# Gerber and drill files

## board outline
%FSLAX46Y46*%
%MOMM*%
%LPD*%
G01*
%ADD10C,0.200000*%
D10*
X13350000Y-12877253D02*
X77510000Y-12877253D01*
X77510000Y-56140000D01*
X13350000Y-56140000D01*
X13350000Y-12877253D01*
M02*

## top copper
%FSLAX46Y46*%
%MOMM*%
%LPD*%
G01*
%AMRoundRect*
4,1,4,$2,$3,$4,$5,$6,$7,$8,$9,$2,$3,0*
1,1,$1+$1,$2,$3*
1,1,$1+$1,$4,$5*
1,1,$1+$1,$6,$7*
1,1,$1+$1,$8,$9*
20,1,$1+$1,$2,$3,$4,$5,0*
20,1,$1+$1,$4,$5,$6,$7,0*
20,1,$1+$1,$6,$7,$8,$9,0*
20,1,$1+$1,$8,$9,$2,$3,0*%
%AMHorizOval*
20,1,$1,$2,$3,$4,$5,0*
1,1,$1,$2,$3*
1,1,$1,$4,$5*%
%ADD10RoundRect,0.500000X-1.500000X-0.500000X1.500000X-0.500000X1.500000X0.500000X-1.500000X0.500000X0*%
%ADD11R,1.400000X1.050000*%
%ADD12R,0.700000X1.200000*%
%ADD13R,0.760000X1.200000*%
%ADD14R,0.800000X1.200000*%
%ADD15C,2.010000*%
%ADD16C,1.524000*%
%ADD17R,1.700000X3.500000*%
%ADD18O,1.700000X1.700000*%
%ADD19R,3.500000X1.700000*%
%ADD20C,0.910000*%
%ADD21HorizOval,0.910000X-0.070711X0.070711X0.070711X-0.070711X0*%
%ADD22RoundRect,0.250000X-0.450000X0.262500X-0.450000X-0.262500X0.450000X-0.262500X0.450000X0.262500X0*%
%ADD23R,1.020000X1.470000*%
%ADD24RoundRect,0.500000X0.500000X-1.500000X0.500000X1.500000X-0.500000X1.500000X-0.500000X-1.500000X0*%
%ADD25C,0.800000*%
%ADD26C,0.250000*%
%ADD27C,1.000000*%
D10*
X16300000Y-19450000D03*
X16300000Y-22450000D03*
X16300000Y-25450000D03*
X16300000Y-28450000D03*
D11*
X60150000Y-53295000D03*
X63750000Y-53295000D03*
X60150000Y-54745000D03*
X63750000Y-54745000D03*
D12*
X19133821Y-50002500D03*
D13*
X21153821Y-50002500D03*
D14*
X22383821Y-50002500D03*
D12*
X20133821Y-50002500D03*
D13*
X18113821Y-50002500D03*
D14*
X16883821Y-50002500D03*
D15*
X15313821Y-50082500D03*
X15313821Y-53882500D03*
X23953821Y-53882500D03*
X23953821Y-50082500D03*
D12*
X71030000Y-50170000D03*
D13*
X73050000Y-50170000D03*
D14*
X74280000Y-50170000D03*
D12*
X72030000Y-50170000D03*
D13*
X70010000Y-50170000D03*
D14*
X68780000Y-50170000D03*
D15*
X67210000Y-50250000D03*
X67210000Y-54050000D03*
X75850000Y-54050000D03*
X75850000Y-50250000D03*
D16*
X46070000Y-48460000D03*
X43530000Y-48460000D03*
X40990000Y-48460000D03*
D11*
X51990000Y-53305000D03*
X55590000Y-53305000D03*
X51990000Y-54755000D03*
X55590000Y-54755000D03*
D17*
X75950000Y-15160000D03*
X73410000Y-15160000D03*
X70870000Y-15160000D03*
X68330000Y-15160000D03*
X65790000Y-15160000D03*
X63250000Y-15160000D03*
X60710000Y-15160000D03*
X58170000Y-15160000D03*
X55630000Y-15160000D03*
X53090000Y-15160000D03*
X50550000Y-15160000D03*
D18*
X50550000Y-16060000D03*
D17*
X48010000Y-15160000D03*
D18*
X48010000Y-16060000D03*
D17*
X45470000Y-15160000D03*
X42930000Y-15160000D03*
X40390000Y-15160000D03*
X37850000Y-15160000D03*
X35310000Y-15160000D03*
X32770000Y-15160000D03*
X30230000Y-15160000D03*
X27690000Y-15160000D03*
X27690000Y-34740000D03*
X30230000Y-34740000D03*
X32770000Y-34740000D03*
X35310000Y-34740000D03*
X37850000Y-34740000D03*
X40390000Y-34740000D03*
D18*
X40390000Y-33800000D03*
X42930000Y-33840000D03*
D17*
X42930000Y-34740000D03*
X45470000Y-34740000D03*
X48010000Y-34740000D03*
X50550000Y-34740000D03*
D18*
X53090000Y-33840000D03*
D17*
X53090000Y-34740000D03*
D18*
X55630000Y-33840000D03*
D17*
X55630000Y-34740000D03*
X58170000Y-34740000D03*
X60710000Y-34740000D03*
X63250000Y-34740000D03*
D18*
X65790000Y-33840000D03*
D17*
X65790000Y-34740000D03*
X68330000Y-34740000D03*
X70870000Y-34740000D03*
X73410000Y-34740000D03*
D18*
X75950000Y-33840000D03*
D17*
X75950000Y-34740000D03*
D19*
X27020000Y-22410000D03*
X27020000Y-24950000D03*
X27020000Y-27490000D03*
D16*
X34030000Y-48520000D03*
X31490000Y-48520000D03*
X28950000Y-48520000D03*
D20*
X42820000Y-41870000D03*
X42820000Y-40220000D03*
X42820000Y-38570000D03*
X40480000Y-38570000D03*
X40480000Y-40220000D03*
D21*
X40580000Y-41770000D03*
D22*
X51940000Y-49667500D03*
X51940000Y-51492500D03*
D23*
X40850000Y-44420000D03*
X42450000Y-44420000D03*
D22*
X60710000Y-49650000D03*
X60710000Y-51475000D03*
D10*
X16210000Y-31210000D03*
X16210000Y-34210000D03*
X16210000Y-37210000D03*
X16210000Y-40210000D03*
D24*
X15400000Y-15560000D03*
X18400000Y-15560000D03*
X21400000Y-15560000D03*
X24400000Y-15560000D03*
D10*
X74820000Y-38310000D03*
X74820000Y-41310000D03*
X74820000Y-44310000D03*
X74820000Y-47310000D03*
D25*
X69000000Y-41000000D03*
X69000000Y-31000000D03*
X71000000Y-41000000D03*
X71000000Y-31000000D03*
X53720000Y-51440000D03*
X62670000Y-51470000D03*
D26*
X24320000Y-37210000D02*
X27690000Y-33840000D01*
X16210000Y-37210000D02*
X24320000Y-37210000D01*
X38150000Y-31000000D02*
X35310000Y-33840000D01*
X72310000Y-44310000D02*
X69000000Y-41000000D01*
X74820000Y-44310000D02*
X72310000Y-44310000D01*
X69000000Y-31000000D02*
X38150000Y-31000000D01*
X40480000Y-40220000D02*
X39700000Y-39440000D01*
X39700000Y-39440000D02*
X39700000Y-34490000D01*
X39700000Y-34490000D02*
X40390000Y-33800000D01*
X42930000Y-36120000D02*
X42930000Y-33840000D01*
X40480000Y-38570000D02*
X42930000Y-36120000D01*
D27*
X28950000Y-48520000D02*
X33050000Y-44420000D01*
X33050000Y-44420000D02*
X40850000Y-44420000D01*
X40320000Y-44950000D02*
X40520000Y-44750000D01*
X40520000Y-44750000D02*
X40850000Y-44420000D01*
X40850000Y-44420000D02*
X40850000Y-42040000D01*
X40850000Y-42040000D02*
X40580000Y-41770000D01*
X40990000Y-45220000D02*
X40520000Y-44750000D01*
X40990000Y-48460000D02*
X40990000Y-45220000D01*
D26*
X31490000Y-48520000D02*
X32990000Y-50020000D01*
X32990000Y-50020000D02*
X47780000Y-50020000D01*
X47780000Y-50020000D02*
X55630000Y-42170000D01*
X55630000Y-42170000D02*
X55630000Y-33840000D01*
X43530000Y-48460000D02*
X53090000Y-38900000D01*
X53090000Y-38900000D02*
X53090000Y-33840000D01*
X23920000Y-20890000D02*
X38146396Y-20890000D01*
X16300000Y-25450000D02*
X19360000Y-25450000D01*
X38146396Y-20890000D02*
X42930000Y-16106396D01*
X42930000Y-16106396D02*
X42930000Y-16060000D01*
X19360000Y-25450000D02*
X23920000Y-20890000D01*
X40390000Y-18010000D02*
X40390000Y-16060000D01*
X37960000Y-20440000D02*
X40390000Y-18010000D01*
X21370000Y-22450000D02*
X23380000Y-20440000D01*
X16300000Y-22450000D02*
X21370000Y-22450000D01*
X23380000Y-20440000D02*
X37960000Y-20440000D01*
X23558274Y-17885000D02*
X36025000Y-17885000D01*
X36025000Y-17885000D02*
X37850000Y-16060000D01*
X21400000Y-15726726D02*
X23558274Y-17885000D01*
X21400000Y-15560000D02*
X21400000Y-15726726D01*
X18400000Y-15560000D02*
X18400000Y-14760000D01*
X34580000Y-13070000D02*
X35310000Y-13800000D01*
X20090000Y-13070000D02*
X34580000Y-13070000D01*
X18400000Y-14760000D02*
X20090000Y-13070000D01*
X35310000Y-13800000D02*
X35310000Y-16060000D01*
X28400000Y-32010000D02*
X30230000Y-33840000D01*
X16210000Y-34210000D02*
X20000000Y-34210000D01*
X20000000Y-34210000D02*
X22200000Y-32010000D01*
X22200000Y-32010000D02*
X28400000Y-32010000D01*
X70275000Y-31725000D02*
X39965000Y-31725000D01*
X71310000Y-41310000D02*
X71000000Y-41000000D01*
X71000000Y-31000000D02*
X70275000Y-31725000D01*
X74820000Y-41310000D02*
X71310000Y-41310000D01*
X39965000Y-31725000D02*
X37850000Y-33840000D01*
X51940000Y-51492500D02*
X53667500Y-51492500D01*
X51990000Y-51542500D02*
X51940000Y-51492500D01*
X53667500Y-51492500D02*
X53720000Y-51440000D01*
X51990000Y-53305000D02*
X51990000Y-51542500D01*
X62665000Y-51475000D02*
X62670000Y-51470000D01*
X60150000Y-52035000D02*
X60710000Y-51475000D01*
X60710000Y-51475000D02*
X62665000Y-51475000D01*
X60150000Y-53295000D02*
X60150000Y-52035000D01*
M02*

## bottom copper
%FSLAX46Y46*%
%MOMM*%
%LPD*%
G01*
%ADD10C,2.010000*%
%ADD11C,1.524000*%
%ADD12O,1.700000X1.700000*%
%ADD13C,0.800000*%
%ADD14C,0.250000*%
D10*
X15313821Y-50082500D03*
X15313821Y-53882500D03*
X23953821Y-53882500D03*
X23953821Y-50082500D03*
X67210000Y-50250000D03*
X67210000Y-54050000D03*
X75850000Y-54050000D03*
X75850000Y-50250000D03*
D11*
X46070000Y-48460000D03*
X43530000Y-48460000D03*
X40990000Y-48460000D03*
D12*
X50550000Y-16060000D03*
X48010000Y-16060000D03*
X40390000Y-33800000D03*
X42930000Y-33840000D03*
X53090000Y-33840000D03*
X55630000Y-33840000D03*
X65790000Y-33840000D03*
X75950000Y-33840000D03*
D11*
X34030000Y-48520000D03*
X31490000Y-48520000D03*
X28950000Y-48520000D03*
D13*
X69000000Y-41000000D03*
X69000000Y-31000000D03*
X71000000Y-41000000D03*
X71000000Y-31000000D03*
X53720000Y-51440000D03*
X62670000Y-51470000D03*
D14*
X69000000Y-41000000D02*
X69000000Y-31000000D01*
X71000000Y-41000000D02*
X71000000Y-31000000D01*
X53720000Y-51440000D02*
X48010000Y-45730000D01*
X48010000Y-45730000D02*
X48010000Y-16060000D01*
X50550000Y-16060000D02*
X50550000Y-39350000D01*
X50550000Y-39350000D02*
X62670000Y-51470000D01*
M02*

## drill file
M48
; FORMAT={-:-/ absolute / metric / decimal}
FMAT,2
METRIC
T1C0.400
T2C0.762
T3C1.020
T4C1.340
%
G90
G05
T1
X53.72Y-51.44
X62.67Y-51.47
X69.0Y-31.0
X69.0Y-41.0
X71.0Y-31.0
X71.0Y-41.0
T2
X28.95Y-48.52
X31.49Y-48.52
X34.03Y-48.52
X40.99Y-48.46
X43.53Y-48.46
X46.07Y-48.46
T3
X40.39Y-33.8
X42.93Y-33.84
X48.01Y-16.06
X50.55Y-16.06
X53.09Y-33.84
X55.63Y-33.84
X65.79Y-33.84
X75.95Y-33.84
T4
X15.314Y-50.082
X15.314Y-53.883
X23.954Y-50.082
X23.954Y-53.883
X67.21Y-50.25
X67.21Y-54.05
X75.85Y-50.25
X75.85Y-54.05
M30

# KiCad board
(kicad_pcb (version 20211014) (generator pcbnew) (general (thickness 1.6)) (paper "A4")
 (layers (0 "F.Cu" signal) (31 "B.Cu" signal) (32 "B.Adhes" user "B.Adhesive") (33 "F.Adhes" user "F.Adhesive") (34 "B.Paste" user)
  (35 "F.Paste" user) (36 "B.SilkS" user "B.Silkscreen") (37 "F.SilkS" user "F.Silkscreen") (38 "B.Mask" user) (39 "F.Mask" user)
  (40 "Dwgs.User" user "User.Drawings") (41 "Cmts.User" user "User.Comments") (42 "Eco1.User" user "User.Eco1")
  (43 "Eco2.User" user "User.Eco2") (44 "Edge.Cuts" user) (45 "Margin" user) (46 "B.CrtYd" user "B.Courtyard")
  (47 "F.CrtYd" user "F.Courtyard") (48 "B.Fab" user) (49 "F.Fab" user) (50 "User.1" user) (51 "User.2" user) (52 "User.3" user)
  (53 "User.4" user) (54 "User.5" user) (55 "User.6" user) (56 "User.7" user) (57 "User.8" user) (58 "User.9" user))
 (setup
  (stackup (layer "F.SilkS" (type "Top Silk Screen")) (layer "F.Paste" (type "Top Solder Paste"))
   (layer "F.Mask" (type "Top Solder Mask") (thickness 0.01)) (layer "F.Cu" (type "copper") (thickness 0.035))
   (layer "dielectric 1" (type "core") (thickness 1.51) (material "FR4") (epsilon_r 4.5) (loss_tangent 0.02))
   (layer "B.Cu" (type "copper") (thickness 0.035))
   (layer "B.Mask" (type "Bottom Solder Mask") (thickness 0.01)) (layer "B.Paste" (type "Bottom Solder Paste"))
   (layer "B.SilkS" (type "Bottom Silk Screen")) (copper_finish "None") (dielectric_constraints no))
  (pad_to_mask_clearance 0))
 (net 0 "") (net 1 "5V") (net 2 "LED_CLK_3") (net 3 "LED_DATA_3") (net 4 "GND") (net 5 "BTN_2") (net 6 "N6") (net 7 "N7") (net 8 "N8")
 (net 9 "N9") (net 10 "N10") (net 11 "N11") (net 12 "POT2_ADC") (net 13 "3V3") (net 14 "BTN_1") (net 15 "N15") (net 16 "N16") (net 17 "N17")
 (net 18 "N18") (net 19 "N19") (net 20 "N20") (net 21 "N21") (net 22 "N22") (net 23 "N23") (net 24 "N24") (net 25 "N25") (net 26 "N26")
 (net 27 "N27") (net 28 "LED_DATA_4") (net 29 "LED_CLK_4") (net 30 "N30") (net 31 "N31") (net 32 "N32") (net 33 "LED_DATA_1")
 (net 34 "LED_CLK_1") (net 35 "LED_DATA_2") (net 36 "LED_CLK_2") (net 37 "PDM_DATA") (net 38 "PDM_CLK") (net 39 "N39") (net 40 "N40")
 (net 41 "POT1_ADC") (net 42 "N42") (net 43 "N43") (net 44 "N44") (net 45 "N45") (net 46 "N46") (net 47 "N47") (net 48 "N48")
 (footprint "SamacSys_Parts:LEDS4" (layer "F.Cu") (at 16.3 19.45)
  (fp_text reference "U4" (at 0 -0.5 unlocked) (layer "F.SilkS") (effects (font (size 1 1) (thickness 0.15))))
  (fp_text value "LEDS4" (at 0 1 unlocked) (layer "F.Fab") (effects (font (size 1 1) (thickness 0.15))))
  (pad "1" smd roundrect (at 0 0) (size 4 2) (layers "F.Cu" "F.Paste" "F.Mask") (roundrect_rratio 0.25) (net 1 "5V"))
  (pad "2" smd roundrect (at 0 3) (size 4 2) (layers "F.Cu" "F.Paste" "F.Mask") (roundrect_rratio 0.25) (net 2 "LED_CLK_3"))
  (pad "3" smd roundrect (at 0 6) (size 4 2) (layers "F.Cu" "F.Paste" "F.Mask") (roundrect_rratio 0.25) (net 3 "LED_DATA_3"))
  (pad "4" smd roundrect (at 0 9) (size 4 2) (layers "F.Cu" "F.Paste" "F.Mask") (roundrect_rratio 0.25) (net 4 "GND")))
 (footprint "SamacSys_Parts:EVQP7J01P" (layer "F.Cu") (at 61.65 54.02)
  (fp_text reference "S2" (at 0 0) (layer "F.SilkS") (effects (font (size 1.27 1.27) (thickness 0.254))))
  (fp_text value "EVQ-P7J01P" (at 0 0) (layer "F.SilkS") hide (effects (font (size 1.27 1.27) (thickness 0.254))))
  (pad "1" smd rect locked (at -1.5 -0.725 90) (size 1.05 1.4) (layers "F.Cu" "F.Paste" "F.Mask") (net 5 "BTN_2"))
  (pad "2" smd rect locked (at 2.1 -0.725 90) (size 1.05 1.4) (layers "F.Cu" "F.Paste" "F.Mask") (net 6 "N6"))
  (pad "3" smd rect locked (at -1.5 0.725 90) (size 1.05 1.4) (layers "F.Cu" "F.Paste" "F.Mask") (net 4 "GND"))
  (pad "4" smd rect locked (at 2.1 0.725 90) (size 1.05 1.4) (layers "F.Cu" "F.Paste" "F.Mask") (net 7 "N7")))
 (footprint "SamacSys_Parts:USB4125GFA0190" (layer "F.Cu") (at 19.633821 53.0825)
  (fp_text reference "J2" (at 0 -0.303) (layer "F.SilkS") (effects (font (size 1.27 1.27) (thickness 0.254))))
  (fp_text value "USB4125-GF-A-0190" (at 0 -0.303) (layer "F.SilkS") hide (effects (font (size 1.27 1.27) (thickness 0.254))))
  (pad "A5" smd rect locked (at -0.5 -3.08) (size 0.7 1.2) (layers "F.Cu" "F.Paste" "F.Mask") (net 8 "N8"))
  (pad "A9" smd rect locked (at 1.52 -3.08) (size 0.76 1.2) (layers "F.Cu" "F.Paste" "F.Mask") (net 1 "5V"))
  (pad "A12" smd rect locked (at 2.75 -3.08) (size 0.8 1.2) (layers "F.Cu" "F.Paste" "F.Mask") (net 4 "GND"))
  (pad "B5" smd rect locked (at 0.5 -3.08) (size 0.7 1.2) (layers "F.Cu" "F.Paste" "F.Mask") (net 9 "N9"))
  (pad "B9" smd rect locked (at -1.52 -3.08) (size 0.76 1.2) (layers "F.Cu" "F.Paste" "F.Mask") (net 1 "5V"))
  (pad "B12" smd rect locked (at -2.75 -3.08) (size 0.8 1.2) (layers "F.Cu" "F.Paste" "F.Mask") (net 4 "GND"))
  (pad "MH1" thru_hole circle locked (at -4.32 -3) (size 2.01 2.01) (drill 1.34) (layers *.Cu *.Mask) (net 4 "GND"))
  (pad "MH2" thru_hole circle locked (at -4.32 0.8) (size 2.01 2.01) (drill 1.34) (layers *.Cu *.Mask) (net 4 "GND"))
  (pad "MH3" thru_hole circle locked (at 4.32 0.8) (size 2.01 2.01) (drill 1.34) (layers *.Cu *.Mask) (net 4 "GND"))
  (pad "MH4" thru_hole circle locked (at 4.32 -3) (size 2.01 2.01) (drill 1.34) (layers *.Cu *.Mask) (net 4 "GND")))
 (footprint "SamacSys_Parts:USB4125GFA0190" (layer "F.Cu") (at 71.53 53.25)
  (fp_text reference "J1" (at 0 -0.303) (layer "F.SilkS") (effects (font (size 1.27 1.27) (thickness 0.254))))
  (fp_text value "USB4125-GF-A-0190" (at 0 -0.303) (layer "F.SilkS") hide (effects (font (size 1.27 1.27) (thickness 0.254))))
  (pad "A5" smd rect locked (at -0.5 -3.08) (size 0.7 1.2) (layers "F.Cu" "F.Paste" "F.Mask") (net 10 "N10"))
  (pad "A9" smd rect locked (at 1.52 -3.08) (size 0.76 1.2) (layers "F.Cu" "F.Paste" "F.Mask") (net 1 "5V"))
  (pad "A12" smd rect locked (at 2.75 -3.08) (size 0.8 1.2) (layers "F.Cu" "F.Paste" "F.Mask") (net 4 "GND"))
  (pad "B5" smd rect locked (at 0.5 -3.08) (size 0.7 1.2) (layers "F.Cu" "F.Paste" "F.Mask") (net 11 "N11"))
  (pad "B9" smd rect locked (at -1.52 -3.08) (size 0.76 1.2) (layers "F.Cu" "F.Paste" "F.Mask") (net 1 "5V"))
  (pad "B12" smd rect locked (at -2.75 -3.08) (size 0.8 1.2) (layers "F.Cu" "F.Paste" "F.Mask") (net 4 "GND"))
  (pad "MH1" thru_hole circle locked (at -4.32 -3) (size 2.01 2.01) (drill 1.34) (layers *.Cu *.Mask) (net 4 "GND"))
  (pad "MH2" thru_hole circle locked (at -4.32 0.8) (size 2.01 2.01) (drill 1.34) (layers *.Cu *.Mask) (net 4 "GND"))
  (pad "MH3" thru_hole circle locked (at 4.32 0.8) (size 2.01 2.01) (drill 1.34) (layers *.Cu *.Mask) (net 4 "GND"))
  (pad "MH4" thru_hole circle locked (at 4.32 -3) (size 2.01 2.01) (drill 1.34) (layers *.Cu *.Mask) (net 4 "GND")))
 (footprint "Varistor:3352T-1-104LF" (layer "F.Cu") (at 43.53 48.46 180)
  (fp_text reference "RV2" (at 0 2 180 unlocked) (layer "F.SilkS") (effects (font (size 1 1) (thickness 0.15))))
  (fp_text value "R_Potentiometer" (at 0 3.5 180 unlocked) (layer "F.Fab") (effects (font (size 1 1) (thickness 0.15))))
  (pad "1" thru_hole circle (at -2.54 0 180) (size 1.524 1.524) (drill 0.762) (layers *.Cu *.Mask) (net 4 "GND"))
  (pad "2" thru_hole circle (at 0 0 180) (size 1.524 1.524) (drill 0.762) (layers *.Cu *.Mask) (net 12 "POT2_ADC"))
  (pad "3" thru_hole circle (at 2.54 0 180) (size 1.524 1.524) (drill 0.762) (layers *.Cu *.Mask) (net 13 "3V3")))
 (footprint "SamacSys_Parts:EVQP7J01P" (layer "F.Cu") (at 53.49 54.03)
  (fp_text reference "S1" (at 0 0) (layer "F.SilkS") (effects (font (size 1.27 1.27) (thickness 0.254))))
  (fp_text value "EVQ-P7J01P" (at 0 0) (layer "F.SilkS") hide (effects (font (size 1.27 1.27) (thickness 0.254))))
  (pad "1" smd rect locked (at -1.5 -0.725 90) (size 1.05 1.4) (layers "F.Cu" "F.Paste" "F.Mask") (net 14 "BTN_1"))
  (pad "2" smd rect locked (at 2.1 -0.725 90) (size 1.05 1.4) (layers "F.Cu" "F.Paste" "F.Mask") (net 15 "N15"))
  (pad "3" smd rect locked (at -1.5 0.725 90) (size 1.05 1.4) (layers "F.Cu" "F.Paste" "F.Mask") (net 4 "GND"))
  (pad "4" smd rect locked (at 2.1 0.725 90) (size 1.05 1.4) (layers "F.Cu" "F.Paste" "F.Mask") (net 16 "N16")))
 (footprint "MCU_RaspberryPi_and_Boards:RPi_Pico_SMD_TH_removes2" (layer "F.Cu") (at 51.82 24.95 -90)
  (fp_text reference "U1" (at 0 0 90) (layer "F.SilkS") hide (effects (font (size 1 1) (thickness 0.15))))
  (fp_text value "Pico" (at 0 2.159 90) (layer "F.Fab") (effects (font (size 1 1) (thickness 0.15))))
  (pad "1" smd rect (at -8.89 -24.13 270) (size 3.5 1.7) (drill (offset -0.9 0)) (layers "F.Cu" "F.Mask") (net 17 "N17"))
  (pad "2" smd rect (at -8.89 -21.59 270) (size 3.5 1.7) (drill (offset -0.9 0)) (layers "F.Cu" "F.Mask") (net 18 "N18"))
  (pad "3" smd rect (at -8.89 -19.05 270) (size 3.5 1.7) (drill (offset -0.9 0)) (layers "F.Cu" "F.Mask") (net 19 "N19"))
  (pad "4" smd rect (at -8.89 -16.51 270) (size 3.5 1.7) (drill (offset -0.9 0)) (layers "F.Cu" "F.Mask") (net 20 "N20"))
  (pad "5" smd rect (at -8.89 -13.97 270) (size 3.5 1.7) (drill (offset -0.9 0)) (layers "F.Cu" "F.Mask") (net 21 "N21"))
  (pad "6" smd rect (at -8.89 -11.43 270) (size 3.5 1.7) (drill (offset -0.9 0)) (layers "F.Cu" "F.Mask") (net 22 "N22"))
  (pad "7" smd rect (at -8.89 -8.89 270) (size 3.5 1.7) (drill (offset -0.9 0)) (layers "F.Cu" "F.Mask") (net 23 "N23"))
  (pad "8" smd rect (at -8.89 -6.35 270) (size 3.5 1.7) (drill (offset -0.9 0)) (layers "F.Cu" "F.Mask") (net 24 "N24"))
  (pad "9" smd rect (at -8.89 -3.81 270) (size 3.5 1.7) (drill (offset -0.9 0)) (layers "F.Cu" "F.Mask") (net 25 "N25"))
  (pad "10" smd rect (at -8.89 -1.27 270) (size 3.5 1.7) (drill (offset -0.9 0)) (layers "F.Cu" "F.Mask") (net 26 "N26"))
  (pad "11" smd rect (at -8.89 1.27 270) (size 3.5 1.7) (drill (offset -0.9 0)) (layers "F.Cu" "F.Mask") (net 5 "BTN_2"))
  (pad "11" thru_hole oval (at -8.89 1.27 270) (size 1.7 1.7) (drill 1.02) (layers *.Cu *.Mask) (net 5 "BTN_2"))
  (pad "12" smd rect (at -8.89 3.81 270) (size 3.5 1.7) (drill (offset -0.9 0)) (layers "F.Cu" "F.Mask") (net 14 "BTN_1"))
  (pad "12" thru_hole oval (at -8.89 3.81 270) (size 1.7 1.7) (drill 1.02) (layers *.Cu *.Mask) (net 14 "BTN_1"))
  (pad "13" smd rect (at -8.89 6.35 270) (size 3.5 1.7) (drill (offset -0.9 0)) (layers "F.Cu" "F.Mask") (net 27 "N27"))
  (pad "14" smd rect (at -8.89 8.89 270) (size 3.5 1.7) (drill (offset -0.9 0)) (layers "F.Cu" "F.Mask") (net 3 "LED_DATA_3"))
  (pad "15" smd rect (at -8.89 11.43 270) (size 3.5 1.7) (drill (offset -0.9 0)) (layers "F.Cu" "F.Mask") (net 2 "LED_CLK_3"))
  (pad "16" smd rect (at -8.89 13.97 270) (size 3.5 1.7) (drill (offset -0.9 0)) (layers "F.Cu" "F.Mask") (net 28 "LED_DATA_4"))
  (pad "17" smd rect (at -8.89 16.51 270) (size 3.5 1.7) (drill (offset -0.9 0)) (layers "F.Cu" "F.Mask") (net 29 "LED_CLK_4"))
  (pad "18" smd rect (at -8.89 19.05 270) (size 3.5 1.7) (drill (offset -0.9 0)) (layers "F.Cu" "F.Mask") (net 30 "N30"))
  (pad "19" smd rect (at -8.89 21.59 270) (size 3.5 1.7) (drill (offset -0.9 0)) (layers "F.Cu" "F.Mask") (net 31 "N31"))
  (pad "20" smd rect (at -8.89 24.13 270) (size 3.5 1.7) (drill (offset -0.9 0)) (layers "F.Cu" "F.Mask") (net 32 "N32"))
  (pad "21" smd rect (at 8.89 24.13 270) (size 3.5 1.7) (drill (offset 0.9 0)) (layers "F.Cu" "F.Mask") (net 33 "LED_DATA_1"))
  (pad "22" smd rect (at 8.89 21.59 270) (size 3.5 1.7) (drill (offset 0.9 0)) (layers "F.Cu" "F.Mask") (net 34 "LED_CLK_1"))
  (pad "23" smd rect (at 8.89 19.05 270) (size 3.5 1.7) (drill (offset 0.9 0)) (layers "F.Cu" "F.Mask") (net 4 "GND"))
  (pad "24" smd rect (at 8.89 16.51 270) (size 3.5 1.7) (drill (offset 0.9 0)) (layers "F.Cu" "F.Mask") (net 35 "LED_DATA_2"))
  (pad "25" smd rect (at 8.89 13.97 270) (size 3.5 1.7) (drill (offset 0.9 0)) (layers "F.Cu" "F.Mask") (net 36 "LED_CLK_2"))
  (pad "26" smd rect (at 8.89 11.43 270) (size 3.5 1.7) (drill (offset 0.9 0)) (layers "F.Cu" "F.Mask") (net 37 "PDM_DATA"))
  (pad "26" thru_hole oval (at 8.85 11.43 270) (size 1.7 1.7) (drill 1.02) (layers *.Cu *.Mask) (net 37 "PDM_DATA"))
  (pad "27" thru_hole oval (at 8.89 8.89 270) (size 1.7 1.7) (drill 1.02) (layers *.Cu *.Mask) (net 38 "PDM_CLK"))
  (pad "27" smd rect (at 8.89 8.89 270) (size 3.5 1.7) (drill (offset 0.9 0)) (layers "F.Cu" "F.Mask") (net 38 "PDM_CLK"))
  (pad "28" smd rect (at 8.89 6.35 270) (size 3.5 1.7) (drill (offset 0.9 0)) (layers "F.Cu" "F.Mask") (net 4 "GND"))
  (pad "29" smd rect (at 8.89 3.81 270) (size 3.5 1.7) (drill (offset 0.9 0)) (layers "F.Cu" "F.Mask") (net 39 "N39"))
  (pad "30" smd rect (at 8.89 1.27 270) (size 3.5 1.7) (drill (offset 0.9 0)) (layers "F.Cu" "F.Mask") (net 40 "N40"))
  (pad "31" thru_hole oval (at 8.89 -1.27 270) (size 1.7 1.7) (drill 1.02) (layers *.Cu *.Mask) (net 12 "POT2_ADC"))
  (pad "31" smd rect (at 8.89 -1.27 270) (size 3.5 1.7) (drill (offset 0.9 0)) (layers "F.Cu" "F.Mask") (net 12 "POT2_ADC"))
  (pad "32" thru_hole oval (at 8.89 -3.81 270) (size 1.7 1.7) (drill 1.02) (layers *.Cu *.Mask) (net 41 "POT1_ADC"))
  (pad "32" smd rect (at 8.89 -3.81 270) (size 3.5 1.7) (drill (offset 0.9 0)) (layers "F.Cu" "F.Mask") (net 41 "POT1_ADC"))
  (pad "33" smd rect (at 8.89 -6.35 270) (size 3.5 1.7) (drill (offset 0.9 0)) (layers "F.Cu" "F.Mask") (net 4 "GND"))
  (pad "34" smd rect (at 8.89 -8.89 270) (size 3.5 1.7) (drill (offset 0.9 0)) (layers "F.Cu" "F.Mask") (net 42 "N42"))
  (pad "35" smd rect (at 8.89 -11.43 270) (size 3.5 1.7) (drill (offset 0.9 0)) (layers "F.Cu" "F.Mask") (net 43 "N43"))
  (pad "36" thru_hole oval (at 8.89 -13.97 270) (size 1.7 1.7) (drill 1.02) (layers *.Cu *.Mask) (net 13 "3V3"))
  (pad "36" smd rect (at 8.89 -13.97 270) (size 3.5 1.7) (drill (offset 0.9 0)) (layers "F.Cu" "F.Mask") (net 13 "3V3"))
  (pad "37" smd rect (at 8.89 -16.51 270) (size 3.5 1.7) (drill (offset 0.9 0)) (layers "F.Cu" "F.Mask") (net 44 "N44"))
  (pad "38" smd rect (at 8.89 -19.05 270) (size 3.5 1.7) (drill (offset 0.9 0)) (layers "F.Cu" "F.Mask") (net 4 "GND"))
  (pad "39" smd rect (at 8.89 -21.59 270) (size 3.5 1.7) (drill (offset 0.9 0)) (layers "F.Cu" "F.Mask") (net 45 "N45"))
  (pad "40" thru_hole oval (at 8.89 -24.13 270) (size 1.7 1.7) (drill 1.02) (layers *.Cu *.Mask) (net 1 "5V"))
  (pad "40" smd rect (at 8.89 -24.13 270) (size 3.5 1.7) (drill (offset 0.9 0)) (layers "F.Cu" "F.Mask") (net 1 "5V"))
  (pad "41" smd rect (at -2.54 23.9) (size 3.5 1.7) (drill (offset -0.9 0)) (layers "F.Cu" "F.Mask") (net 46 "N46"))
  (pad "42" smd rect (at 0 23.9) (size 3.5 1.7) (drill (offset -0.9 0)) (layers "F.Cu" "F.Mask") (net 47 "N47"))
  (pad "43" smd rect (at 2.54 23.9) (size 3.5 1.7) (drill (offset -0.9 0)) (layers "F.Cu" "F.Mask") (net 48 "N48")))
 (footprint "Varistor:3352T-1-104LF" (layer "F.Cu") (at 31.49 48.52 180)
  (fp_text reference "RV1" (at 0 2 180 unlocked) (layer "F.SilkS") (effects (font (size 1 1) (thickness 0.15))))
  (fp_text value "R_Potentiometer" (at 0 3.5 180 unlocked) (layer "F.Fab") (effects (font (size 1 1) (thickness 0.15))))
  (pad "1" thru_hole circle (at -2.54 0 180) (size 1.524 1.524) (drill 0.762) (layers *.Cu *.Mask) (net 4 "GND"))
  (pad "2" thru_hole circle (at 0 0 180) (size 1.524 1.524) (drill 0.762) (layers *.Cu *.Mask) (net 41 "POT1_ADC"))
  (pad "3" thru_hole circle (at 2.54 0 180) (size 1.524 1.524) (drill 0.762) (layers *.Cu *.Mask) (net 13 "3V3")))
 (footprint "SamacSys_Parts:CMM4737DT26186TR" (layer "F.Cu") (at 41.65 40.22 180)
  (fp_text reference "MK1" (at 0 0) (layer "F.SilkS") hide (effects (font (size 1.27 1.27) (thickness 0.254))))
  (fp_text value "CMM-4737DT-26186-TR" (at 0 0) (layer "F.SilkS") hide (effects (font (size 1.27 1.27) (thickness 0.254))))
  (pad "1" smd circle locked (at -1.17 -1.65 270) (size 0.91 0.91) (layers "F.Cu" "F.Paste" "F.Mask") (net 4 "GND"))
  (pad "2" smd circle locked (at -1.17 0 270) (size 0.91 0.91) (layers "F.Cu" "F.Paste" "F.Mask") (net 4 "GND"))
  (pad "3" smd circle locked (at -1.17 1.65 270) (size 0.91 0.91) (layers "F.Cu" "F.Paste" "F.Mask") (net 4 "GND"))
  (pad "4" smd circle locked (at 1.17 1.65 270) (size 0.91 0.91) (layers "F.Cu" "F.Paste" "F.Mask") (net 38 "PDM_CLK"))
  (pad "5" smd circle locked (at 1.17 0 270) (size 0.91 0.91) (layers "F.Cu" "F.Paste" "F.Mask") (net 37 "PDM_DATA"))
  (pad "6" smd oval locked (at 1.07 -1.55 225) (size 0.91 1.11) (layers "F.Cu" "F.Paste" "F.Mask") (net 13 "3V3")))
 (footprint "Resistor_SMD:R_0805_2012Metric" (layer "F.Cu") (at 51.94 50.58 -90)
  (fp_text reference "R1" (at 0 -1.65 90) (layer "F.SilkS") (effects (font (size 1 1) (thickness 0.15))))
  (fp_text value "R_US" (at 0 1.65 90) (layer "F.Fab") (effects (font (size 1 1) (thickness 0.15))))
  (pad "1" smd roundrect (at -0.9125 0 270) (size 1.025 1.4) (layers "F.Cu" "F.Paste" "F.Mask") (roundrect_rratio 0.243902) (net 13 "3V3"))
  (pad "2" smd roundrect (at 0.9125 0 270) (size 1.025 1.4) (layers "F.Cu" "F.Paste" "F.Mask") (roundrect_rratio 0.243902) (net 14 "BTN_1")))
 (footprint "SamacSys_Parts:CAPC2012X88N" (layer "F.Cu") (at 41.65 44.42)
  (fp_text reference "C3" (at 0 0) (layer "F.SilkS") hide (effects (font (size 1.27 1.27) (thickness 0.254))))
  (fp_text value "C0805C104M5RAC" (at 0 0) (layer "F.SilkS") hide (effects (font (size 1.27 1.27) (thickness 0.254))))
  (pad "1" smd rect locked (at -0.8 0) (size 1.02 1.47) (layers "F.Cu" "F.Paste" "F.Mask") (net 13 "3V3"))
  (pad "2" smd rect locked (at 0.8 0) (size 1.02 1.47) (layers "F.Cu" "F.Paste" "F.Mask") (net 4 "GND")))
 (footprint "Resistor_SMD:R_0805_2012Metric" (layer "F.Cu") (at 60.71 50.5625 -90)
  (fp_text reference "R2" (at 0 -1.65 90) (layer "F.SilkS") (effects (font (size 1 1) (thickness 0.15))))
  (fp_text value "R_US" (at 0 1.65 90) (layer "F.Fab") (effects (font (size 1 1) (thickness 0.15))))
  (pad "1" smd roundrect (at -0.9125 0 270) (size 1.025 1.4) (layers "F.Cu" "F.Paste" "F.Mask") (roundrect_rratio 0.243902) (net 13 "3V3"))
  (pad "2" smd roundrect (at 0.9125 0 270) (size 1.025 1.4) (layers "F.Cu" "F.Paste" "F.Mask") (roundrect_rratio 0.243902) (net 5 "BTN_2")))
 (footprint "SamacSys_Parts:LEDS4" (layer "F.Cu") (at 16.21 31.21)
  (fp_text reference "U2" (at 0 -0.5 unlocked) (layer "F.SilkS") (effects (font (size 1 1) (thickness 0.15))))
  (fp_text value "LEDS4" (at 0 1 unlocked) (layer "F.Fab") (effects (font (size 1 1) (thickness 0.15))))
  (pad "1" smd roundrect (at 0 0) (size 4 2) (layers "F.Cu" "F.Paste" "F.Mask") (roundrect_rratio 0.25) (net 1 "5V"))
  (pad "2" smd roundrect (at 0 3) (size 4 2) (layers "F.Cu" "F.Paste" "F.Mask") (roundrect_rratio 0.25) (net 34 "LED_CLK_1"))
  (pad "3" smd roundrect (at 0 6) (size 4 2) (layers "F.Cu" "F.Paste" "F.Mask") (roundrect_rratio 0.25) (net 33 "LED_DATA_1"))
  (pad "4" smd roundrect (at 0 9) (size 4 2) (layers "F.Cu" "F.Paste" "F.Mask") (roundrect_rratio 0.25) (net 4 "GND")))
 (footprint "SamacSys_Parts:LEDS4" (layer "F.Cu") (at 15.4 15.56 90)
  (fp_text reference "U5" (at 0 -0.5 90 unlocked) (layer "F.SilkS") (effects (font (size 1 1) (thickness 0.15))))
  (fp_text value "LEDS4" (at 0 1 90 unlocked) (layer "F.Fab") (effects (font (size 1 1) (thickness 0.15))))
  (pad "1" smd roundrect (at 0 0 90) (size 4 2) (layers "F.Cu" "F.Paste" "F.Mask") (roundrect_rratio 0.25) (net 1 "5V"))
  (pad "2" smd roundrect (at 0 3 90) (size 4 2) (layers "F.Cu" "F.Paste" "F.Mask") (roundrect_rratio 0.25) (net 29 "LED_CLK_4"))
  (pad "3" smd roundrect (at 0 6 90) (size 4 2) (layers "F.Cu" "F.Paste" "F.Mask") (roundrect_rratio 0.25) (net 28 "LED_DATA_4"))
  (pad "4" smd roundrect (at 0 9 90) (size 4 2) (layers "F.Cu" "F.Paste" "F.Mask") (roundrect_rratio 0.25) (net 4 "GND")))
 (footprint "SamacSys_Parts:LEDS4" (layer "F.Cu") (at 74.82 38.31)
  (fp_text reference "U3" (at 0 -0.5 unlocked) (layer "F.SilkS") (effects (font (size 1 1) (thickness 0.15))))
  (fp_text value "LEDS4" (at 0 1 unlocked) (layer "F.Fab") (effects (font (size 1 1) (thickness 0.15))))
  (pad "1" smd roundrect (at 0 0) (size 4 2) (layers "F.Cu" "F.Paste" "F.Mask") (roundrect_rratio 0.25) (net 1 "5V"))
  (pad "2" smd roundrect (at 0 3) (size 4 2) (layers "F.Cu" "F.Paste" "F.Mask") (roundrect_rratio 0.25) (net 36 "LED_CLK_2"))
  (pad "3" smd roundrect (at 0 6) (size 4 2) (layers "F.Cu" "F.Paste" "F.Mask") (roundrect_rratio 0.25) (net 35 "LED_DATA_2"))
  (pad "4" smd roundrect (at 0 9) (size 4 2) (layers "F.Cu" "F.Paste" "F.Mask") (roundrect_rratio 0.25) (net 4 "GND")))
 (gr_rect (start 13.35 12.877253) (end 77.51 56.14) (layer "Edge.Cuts") (width 0.2) (fill none))
 (segment (start 24.32 37.21) (end 27.69 33.84) (width 0.25) (layer "F.Cu") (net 33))
 (segment (start 16.21 37.21) (end 24.32 37.21) (width 0.25) (layer "F.Cu") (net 33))
 (segment (start 38.15 31) (end 35.31 33.84) (width 0.25) (layer "F.Cu") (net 35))
 (segment (start 72.31 44.31) (end 69 41) (width 0.25) (layer "F.Cu") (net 35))
 (segment (start 74.82 44.31) (end 72.31 44.31) (width 0.25) (layer "F.Cu") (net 35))
 (segment (start 69 31) (end 38.15 31) (width 0.25) (layer "F.Cu") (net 35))
 (via (at 69 41) (size 0.8) (drill 0.4) (layers "F.Cu" "B.Cu") (free) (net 35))
 (via (at 69 31) (size 0.8) (drill 0.4) (layers "F.Cu" "B.Cu") (free) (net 35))
 (segment (start 69 41) (end 69 31) (width 0.25) (layer "B.Cu") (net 35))
 (segment (start 40.48 40.22) (end 39.7 39.44) (width 0.25) (layer "F.Cu") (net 37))
 (segment (start 39.7 39.44) (end 39.7 34.49) (width 0.25) (layer "F.Cu") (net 37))
 (segment (start 39.7 34.49) (end 40.39 33.8) (width 0.25) (layer "F.Cu") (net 37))
 (segment (start 42.93 36.12) (end 42.93 33.84) (width 0.25) (layer "F.Cu") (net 38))
 (segment (start 40.48 38.57) (end 42.93 36.12) (width 0.25) (layer "F.Cu") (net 38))
 (segment (start 28.95 48.52) (end 33.05 44.42) (width 1) (layer "F.Cu") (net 13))
 (segment (start 33.05 44.42) (end 40.85 44.42) (width 1) (layer "F.Cu") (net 13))
 (segment (start 40.32 44.95) (end 40.52 44.75) (width 1) (layer "F.Cu") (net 13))
 (segment (start 40.52 44.75) (end 40.85 44.42) (width 1) (layer "F.Cu") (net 13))
 (segment (start 40.85 44.42) (end 40.85 42.04) (width 1) (layer "F.Cu") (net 13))
 (segment (start 40.85 42.04) (end 40.58 41.77) (width 1) (layer "F.Cu") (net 13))
 (segment (start 40.99 45.22) (end 40.52 44.75) (width 1) (layer "F.Cu") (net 13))
 (segment (start 40.99 48.46) (end 40.99 45.22) (width 1) (layer "F.Cu") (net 13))
 (segment (start 31.49 48.52) (end 32.99 50.02) (width 0.25) (layer "F.Cu") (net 41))
 (segment (start 32.99 50.02) (end 47.78 50.02) (width 0.25) (layer "F.Cu") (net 41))
 (segment (start 47.78 50.02) (end 55.63 42.17) (width 0.25) (layer "F.Cu") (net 41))
 (segment (start 55.63 42.17) (end 55.63 33.84) (width 0.25) (layer "F.Cu") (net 41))
 (segment (start 43.53 48.46) (end 53.09 38.9) (width 0.25) (layer "F.Cu") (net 12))
 (segment (start 53.09 38.9) (end 53.09 33.84) (width 0.25) (layer "F.Cu") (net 12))
 (segment (start 23.92 20.89) (end 38.146396 20.89) (width 0.25) (layer "F.Cu") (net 3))
 (segment (start 16.3 25.45) (end 19.36 25.45) (width 0.25) (layer "F.Cu") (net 3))
 (segment (start 38.146396 20.89) (end 42.93 16.106396) (width 0.25) (layer "F.Cu") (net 3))
 (segment (start 42.93 16.106396) (end 42.93 16.06) (width 0.25) (layer "F.Cu") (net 3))
 (segment (start 19.36 25.45) (end 23.92 20.89) (width 0.25) (layer "F.Cu") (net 3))
 (segment (start 40.39 18.01) (end 40.39 16.06) (width 0.25) (layer "F.Cu") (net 2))
 (segment (start 37.96 20.44) (end 40.39 18.01) (width 0.25) (layer "F.Cu") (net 2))
 (segment (start 21.37 22.45) (end 23.38 20.44) (width 0.25) (layer "F.Cu") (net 2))
 (segment (start 16.3 22.45) (end 21.37 22.45) (width 0.25) (layer "F.Cu") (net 2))
 (segment (start 23.38 20.44) (end 37.96 20.44) (width 0.25) (layer "F.Cu") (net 2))
 (segment (start 23.558274 17.885) (end 36.025 17.885) (width 0.25) (layer "F.Cu") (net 28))
 (segment (start 36.025 17.885) (end 37.85 16.06) (width 0.25) (layer "F.Cu") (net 28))
 (segment (start 21.4 15.726726) (end 23.558274 17.885) (width 0.25) (layer "F.Cu") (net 28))
 (segment (start 21.4 15.56) (end 21.4 15.726726) (width 0.25) (layer "F.Cu") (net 28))
 (segment (start 18.4 15.56) (end 18.4 14.76) (width 0.25) (layer "F.Cu") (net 29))
 (segment (start 34.58 13.07) (end 35.31 13.8) (width 0.25) (layer "F.Cu") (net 29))
 (segment (start 20.09 13.07) (end 34.58 13.07) (width 0.25) (layer "F.Cu") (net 29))
 (segment (start 18.4 14.76) (end 20.09 13.07) (width 0.25) (layer "F.Cu") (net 29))
 (segment (start 35.31 13.8) (end 35.31 16.06) (width 0.25) (layer "F.Cu") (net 29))
 (segment (start 28.4 32.01) (end 30.23 33.84) (width 0.25) (layer "F.Cu") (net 34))
 (segment (start 16.21 34.21) (end 20 34.21) (width 0.25) (layer "F.Cu") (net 34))
 (segment (start 20 34.21) (end 22.2 32.01) (width 0.25) (layer "F.Cu") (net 34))
 (segment (start 22.2 32.01) (end 28.4 32.01) (width 0.25) (layer "F.Cu") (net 34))
 (segment (start 70.275 31.725) (end 39.965 31.725) (width 0.25) (layer "F.Cu") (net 36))
 (segment (start 71.31 41.31) (end 71 41) (width 0.25) (layer "F.Cu") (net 36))
 (segment (start 71 31) (end 70.275 31.725) (width 0.25) (layer "F.Cu") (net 36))
 (segment (start 74.82 41.31) (end 71.31 41.31) (width 0.25) (layer "F.Cu") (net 36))
 (segment (start 39.965 31.725) (end 37.85 33.84) (width 0.25) (layer "F.Cu") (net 36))
 (via (at 71 41) (size 0.8) (drill 0.4) (layers "F.Cu" "B.Cu") (free) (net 36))
 (via (at 71 31) (size 0.8) (drill 0.4) (layers "F.Cu" "B.Cu") (free) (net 36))
 (segment (start 71 41) (end 71 31) (width 0.25) (layer "B.Cu") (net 36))
 (segment (start 51.94 51.4925) (end 53.6675 51.4925) (width 0.25) (layer "F.Cu") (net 14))
 (segment (start 51.99 51.5425) (end 51.94 51.4925) (width 0.25) (layer "F.Cu") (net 14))
 (segment (start 53.6675 51.4925) (end 53.72 51.44) (width 0.25) (layer "F.Cu") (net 14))
 (segment (start 51.99 53.305) (end 51.99 51.5425) (width 0.25) (layer "F.Cu") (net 14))
 (via (at 53.72 51.44) (size 0.8) (drill 0.4) (layers "F.Cu" "B.Cu") (free) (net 14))
 (segment (start 53.72 51.44) (end 48.01 45.73) (width 0.25) (layer "B.Cu") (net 14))
 (segment (start 48.01 45.73) (end 48.01 16.06) (width 0.25) (layer "B.Cu") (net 14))
 (segment (start 62.665 51.475) (end 62.67 51.47) (width 0.25) (layer "F.Cu") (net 5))
 (segment (start 60.15 52.035) (end 60.71 51.475) (width 0.25) (layer "F.Cu") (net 5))
 (segment (start 60.71 51.475) (end 62.665 51.475) (width 0.25) (layer "F.Cu") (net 5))
 (segment (start 60.15 53.295) (end 60.15 52.035) (width 0.25) (layer "F.Cu") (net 5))
 (via (at 62.67 51.47) (size 0.8) (drill 0.4) (layers "F.Cu" "B.Cu") (free) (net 5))
 (segment (start 50.55 16.06) (end 50.55 39.35) (width 0.25) (layer "B.Cu") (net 5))
 (segment (start 50.55 39.35) (end 62.67 51.47) (width 0.25) (layer "B.Cu") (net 5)))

